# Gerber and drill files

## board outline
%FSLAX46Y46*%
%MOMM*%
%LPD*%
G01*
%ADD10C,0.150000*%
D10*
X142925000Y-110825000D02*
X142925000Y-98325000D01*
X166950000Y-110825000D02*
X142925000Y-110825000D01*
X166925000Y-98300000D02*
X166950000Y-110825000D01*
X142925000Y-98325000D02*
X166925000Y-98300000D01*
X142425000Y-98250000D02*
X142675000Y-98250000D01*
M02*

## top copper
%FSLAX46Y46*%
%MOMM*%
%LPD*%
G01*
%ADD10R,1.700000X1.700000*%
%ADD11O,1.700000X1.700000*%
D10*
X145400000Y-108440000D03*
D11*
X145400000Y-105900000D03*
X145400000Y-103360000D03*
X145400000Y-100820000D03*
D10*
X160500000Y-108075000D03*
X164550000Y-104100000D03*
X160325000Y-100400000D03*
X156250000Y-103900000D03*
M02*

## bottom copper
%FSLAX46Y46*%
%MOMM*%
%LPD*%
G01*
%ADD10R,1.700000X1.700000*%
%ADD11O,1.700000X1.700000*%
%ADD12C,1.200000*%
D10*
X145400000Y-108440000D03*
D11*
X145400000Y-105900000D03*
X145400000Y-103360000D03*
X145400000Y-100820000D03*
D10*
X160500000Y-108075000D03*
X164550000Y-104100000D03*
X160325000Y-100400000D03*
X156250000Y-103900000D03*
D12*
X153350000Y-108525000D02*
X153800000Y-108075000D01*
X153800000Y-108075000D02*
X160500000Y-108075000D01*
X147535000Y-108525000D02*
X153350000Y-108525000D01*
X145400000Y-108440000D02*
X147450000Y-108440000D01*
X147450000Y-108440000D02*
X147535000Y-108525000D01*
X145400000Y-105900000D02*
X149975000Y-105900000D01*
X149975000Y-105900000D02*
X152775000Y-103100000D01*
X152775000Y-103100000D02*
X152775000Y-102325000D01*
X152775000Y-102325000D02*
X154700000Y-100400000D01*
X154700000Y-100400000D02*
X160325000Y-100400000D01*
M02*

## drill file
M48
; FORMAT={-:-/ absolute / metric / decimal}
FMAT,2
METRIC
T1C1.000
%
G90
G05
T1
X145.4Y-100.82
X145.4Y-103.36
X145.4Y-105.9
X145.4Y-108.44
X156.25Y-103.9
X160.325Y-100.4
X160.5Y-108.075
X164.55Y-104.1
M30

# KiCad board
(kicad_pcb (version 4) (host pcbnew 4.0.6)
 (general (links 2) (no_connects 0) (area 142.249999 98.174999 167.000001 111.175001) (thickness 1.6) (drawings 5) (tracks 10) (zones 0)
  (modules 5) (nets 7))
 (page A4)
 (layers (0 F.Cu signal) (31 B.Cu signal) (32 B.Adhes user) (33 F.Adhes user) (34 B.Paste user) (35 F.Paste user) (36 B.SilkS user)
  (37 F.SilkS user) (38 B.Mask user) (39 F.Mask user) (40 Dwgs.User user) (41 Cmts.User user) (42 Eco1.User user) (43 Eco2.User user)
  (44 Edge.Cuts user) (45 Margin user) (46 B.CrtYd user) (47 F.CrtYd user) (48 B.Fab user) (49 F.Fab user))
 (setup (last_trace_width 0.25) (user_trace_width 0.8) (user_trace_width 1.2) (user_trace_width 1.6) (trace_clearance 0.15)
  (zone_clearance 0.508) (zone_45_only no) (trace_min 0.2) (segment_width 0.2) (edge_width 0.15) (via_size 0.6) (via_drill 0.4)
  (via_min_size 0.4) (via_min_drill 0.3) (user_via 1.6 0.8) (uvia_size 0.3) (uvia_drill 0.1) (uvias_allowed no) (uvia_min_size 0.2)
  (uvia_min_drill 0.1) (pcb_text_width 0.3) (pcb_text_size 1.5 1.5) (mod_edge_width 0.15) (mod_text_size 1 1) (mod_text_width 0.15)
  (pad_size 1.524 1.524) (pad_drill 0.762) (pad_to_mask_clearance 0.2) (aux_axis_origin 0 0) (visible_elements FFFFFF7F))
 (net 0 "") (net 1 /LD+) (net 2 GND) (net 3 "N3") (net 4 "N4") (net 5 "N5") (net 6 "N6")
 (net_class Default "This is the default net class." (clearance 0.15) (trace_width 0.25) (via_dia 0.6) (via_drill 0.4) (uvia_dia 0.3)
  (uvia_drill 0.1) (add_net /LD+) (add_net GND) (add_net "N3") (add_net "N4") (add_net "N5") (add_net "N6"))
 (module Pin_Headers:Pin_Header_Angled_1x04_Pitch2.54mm (layer F.Cu) (at 145.4 108.44 180)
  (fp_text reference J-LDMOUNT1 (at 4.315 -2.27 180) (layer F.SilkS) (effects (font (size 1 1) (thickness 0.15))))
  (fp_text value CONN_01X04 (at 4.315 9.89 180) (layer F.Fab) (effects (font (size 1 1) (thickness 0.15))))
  (pad 1 thru_hole rect (at 0 0 180) (size 1.7 1.7) (drill 1) (layers *.Cu *.Mask) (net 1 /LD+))
  (pad 2 thru_hole oval (at 0 2.54 180) (size 1.7 1.7) (drill 1) (layers *.Cu *.Mask) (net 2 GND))
  (pad 3 thru_hole oval (at 0 5.08 180) (size 1.7 1.7) (drill 1) (layers *.Cu *.Mask) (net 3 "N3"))
  (pad 4 thru_hole oval (at 0 7.62 180) (size 1.7 1.7) (drill 1) (layers *.Cu *.Mask) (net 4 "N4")))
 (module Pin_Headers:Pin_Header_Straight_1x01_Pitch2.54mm (layer F.Cu) (at 160.5 108.075)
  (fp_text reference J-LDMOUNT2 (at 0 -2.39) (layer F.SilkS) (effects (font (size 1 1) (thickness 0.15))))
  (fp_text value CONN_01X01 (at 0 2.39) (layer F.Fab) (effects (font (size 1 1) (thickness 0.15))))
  (pad 1 thru_hole rect (at 0 0) (size 1.7 1.7) (drill 1) (layers *.Cu *.Mask) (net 1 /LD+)))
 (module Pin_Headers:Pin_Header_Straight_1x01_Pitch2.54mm (layer F.Cu) (at 164.55 104.1)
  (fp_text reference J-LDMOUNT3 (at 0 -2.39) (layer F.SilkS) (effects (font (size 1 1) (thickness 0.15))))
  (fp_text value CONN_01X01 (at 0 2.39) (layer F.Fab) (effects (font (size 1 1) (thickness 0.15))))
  (pad 1 thru_hole rect (at 0 0) (size 1.7 1.7) (drill 1) (layers *.Cu *.Mask) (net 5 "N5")))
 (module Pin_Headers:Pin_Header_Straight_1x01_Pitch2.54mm (layer F.Cu) (at 160.325 100.4)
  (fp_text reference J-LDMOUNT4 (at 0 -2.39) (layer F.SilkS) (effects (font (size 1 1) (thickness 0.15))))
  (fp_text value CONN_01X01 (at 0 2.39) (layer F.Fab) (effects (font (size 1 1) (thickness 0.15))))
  (pad 1 thru_hole rect (at 0 0) (size 1.7 1.7) (drill 1) (layers *.Cu *.Mask) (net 2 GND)))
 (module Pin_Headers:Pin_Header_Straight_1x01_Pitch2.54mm (layer F.Cu) (at 156.25 103.9)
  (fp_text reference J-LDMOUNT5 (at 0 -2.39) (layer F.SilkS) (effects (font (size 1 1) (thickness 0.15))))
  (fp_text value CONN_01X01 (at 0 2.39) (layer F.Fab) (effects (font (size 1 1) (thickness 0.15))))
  (pad 1 thru_hole rect (at 0 0) (size 1.7 1.7) (drill 1) (layers *.Cu *.Mask) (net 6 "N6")))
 (gr_line (start 142.925 110.825) (end 142.925 98.325) (layer Edge.Cuts) (width 0.15))
 (gr_line (start 166.95 110.825) (end 142.925 110.825) (layer Edge.Cuts) (width 0.15))
 (gr_line (start 166.925 98.3) (end 166.95 110.825) (layer Edge.Cuts) (width 0.15))
 (gr_line (start 142.925 98.325) (end 166.925 98.3) (layer Edge.Cuts) (width 0.15))
 (gr_line (start 142.425 98.25) (end 142.675 98.25) (layer Edge.Cuts) (width 0.15))
 (segment (start 153.35 108.525) (end 153.8 108.075) (width 1.2) (layer B.Cu) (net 1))
 (segment (start 153.8 108.075) (end 160.5 108.075) (width 1.2) (layer B.Cu) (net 1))
 (segment (start 147.535 108.525) (end 153.35 108.525) (width 1.2) (layer B.Cu) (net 1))
 (segment (start 145.4 108.44) (end 147.45 108.44) (width 1.2) (layer B.Cu) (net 1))
 (segment (start 147.45 108.44) (end 147.535 108.525) (width 1.2) (layer B.Cu) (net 1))
 (segment (start 145.4 105.9) (end 149.975 105.9) (width 1.2) (layer B.Cu) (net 2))
 (segment (start 149.975 105.9) (end 152.775 103.1) (width 1.2) (layer B.Cu) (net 2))
 (segment (start 152.775 103.1) (end 152.775 102.325) (width 1.2) (layer B.Cu) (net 2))
 (segment (start 152.775 102.325) (end 154.7 100.4) (width 1.2) (layer B.Cu) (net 2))
 (segment (start 154.7 100.4) (end 160.325 100.4) (width 1.2) (layer B.Cu) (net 2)))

